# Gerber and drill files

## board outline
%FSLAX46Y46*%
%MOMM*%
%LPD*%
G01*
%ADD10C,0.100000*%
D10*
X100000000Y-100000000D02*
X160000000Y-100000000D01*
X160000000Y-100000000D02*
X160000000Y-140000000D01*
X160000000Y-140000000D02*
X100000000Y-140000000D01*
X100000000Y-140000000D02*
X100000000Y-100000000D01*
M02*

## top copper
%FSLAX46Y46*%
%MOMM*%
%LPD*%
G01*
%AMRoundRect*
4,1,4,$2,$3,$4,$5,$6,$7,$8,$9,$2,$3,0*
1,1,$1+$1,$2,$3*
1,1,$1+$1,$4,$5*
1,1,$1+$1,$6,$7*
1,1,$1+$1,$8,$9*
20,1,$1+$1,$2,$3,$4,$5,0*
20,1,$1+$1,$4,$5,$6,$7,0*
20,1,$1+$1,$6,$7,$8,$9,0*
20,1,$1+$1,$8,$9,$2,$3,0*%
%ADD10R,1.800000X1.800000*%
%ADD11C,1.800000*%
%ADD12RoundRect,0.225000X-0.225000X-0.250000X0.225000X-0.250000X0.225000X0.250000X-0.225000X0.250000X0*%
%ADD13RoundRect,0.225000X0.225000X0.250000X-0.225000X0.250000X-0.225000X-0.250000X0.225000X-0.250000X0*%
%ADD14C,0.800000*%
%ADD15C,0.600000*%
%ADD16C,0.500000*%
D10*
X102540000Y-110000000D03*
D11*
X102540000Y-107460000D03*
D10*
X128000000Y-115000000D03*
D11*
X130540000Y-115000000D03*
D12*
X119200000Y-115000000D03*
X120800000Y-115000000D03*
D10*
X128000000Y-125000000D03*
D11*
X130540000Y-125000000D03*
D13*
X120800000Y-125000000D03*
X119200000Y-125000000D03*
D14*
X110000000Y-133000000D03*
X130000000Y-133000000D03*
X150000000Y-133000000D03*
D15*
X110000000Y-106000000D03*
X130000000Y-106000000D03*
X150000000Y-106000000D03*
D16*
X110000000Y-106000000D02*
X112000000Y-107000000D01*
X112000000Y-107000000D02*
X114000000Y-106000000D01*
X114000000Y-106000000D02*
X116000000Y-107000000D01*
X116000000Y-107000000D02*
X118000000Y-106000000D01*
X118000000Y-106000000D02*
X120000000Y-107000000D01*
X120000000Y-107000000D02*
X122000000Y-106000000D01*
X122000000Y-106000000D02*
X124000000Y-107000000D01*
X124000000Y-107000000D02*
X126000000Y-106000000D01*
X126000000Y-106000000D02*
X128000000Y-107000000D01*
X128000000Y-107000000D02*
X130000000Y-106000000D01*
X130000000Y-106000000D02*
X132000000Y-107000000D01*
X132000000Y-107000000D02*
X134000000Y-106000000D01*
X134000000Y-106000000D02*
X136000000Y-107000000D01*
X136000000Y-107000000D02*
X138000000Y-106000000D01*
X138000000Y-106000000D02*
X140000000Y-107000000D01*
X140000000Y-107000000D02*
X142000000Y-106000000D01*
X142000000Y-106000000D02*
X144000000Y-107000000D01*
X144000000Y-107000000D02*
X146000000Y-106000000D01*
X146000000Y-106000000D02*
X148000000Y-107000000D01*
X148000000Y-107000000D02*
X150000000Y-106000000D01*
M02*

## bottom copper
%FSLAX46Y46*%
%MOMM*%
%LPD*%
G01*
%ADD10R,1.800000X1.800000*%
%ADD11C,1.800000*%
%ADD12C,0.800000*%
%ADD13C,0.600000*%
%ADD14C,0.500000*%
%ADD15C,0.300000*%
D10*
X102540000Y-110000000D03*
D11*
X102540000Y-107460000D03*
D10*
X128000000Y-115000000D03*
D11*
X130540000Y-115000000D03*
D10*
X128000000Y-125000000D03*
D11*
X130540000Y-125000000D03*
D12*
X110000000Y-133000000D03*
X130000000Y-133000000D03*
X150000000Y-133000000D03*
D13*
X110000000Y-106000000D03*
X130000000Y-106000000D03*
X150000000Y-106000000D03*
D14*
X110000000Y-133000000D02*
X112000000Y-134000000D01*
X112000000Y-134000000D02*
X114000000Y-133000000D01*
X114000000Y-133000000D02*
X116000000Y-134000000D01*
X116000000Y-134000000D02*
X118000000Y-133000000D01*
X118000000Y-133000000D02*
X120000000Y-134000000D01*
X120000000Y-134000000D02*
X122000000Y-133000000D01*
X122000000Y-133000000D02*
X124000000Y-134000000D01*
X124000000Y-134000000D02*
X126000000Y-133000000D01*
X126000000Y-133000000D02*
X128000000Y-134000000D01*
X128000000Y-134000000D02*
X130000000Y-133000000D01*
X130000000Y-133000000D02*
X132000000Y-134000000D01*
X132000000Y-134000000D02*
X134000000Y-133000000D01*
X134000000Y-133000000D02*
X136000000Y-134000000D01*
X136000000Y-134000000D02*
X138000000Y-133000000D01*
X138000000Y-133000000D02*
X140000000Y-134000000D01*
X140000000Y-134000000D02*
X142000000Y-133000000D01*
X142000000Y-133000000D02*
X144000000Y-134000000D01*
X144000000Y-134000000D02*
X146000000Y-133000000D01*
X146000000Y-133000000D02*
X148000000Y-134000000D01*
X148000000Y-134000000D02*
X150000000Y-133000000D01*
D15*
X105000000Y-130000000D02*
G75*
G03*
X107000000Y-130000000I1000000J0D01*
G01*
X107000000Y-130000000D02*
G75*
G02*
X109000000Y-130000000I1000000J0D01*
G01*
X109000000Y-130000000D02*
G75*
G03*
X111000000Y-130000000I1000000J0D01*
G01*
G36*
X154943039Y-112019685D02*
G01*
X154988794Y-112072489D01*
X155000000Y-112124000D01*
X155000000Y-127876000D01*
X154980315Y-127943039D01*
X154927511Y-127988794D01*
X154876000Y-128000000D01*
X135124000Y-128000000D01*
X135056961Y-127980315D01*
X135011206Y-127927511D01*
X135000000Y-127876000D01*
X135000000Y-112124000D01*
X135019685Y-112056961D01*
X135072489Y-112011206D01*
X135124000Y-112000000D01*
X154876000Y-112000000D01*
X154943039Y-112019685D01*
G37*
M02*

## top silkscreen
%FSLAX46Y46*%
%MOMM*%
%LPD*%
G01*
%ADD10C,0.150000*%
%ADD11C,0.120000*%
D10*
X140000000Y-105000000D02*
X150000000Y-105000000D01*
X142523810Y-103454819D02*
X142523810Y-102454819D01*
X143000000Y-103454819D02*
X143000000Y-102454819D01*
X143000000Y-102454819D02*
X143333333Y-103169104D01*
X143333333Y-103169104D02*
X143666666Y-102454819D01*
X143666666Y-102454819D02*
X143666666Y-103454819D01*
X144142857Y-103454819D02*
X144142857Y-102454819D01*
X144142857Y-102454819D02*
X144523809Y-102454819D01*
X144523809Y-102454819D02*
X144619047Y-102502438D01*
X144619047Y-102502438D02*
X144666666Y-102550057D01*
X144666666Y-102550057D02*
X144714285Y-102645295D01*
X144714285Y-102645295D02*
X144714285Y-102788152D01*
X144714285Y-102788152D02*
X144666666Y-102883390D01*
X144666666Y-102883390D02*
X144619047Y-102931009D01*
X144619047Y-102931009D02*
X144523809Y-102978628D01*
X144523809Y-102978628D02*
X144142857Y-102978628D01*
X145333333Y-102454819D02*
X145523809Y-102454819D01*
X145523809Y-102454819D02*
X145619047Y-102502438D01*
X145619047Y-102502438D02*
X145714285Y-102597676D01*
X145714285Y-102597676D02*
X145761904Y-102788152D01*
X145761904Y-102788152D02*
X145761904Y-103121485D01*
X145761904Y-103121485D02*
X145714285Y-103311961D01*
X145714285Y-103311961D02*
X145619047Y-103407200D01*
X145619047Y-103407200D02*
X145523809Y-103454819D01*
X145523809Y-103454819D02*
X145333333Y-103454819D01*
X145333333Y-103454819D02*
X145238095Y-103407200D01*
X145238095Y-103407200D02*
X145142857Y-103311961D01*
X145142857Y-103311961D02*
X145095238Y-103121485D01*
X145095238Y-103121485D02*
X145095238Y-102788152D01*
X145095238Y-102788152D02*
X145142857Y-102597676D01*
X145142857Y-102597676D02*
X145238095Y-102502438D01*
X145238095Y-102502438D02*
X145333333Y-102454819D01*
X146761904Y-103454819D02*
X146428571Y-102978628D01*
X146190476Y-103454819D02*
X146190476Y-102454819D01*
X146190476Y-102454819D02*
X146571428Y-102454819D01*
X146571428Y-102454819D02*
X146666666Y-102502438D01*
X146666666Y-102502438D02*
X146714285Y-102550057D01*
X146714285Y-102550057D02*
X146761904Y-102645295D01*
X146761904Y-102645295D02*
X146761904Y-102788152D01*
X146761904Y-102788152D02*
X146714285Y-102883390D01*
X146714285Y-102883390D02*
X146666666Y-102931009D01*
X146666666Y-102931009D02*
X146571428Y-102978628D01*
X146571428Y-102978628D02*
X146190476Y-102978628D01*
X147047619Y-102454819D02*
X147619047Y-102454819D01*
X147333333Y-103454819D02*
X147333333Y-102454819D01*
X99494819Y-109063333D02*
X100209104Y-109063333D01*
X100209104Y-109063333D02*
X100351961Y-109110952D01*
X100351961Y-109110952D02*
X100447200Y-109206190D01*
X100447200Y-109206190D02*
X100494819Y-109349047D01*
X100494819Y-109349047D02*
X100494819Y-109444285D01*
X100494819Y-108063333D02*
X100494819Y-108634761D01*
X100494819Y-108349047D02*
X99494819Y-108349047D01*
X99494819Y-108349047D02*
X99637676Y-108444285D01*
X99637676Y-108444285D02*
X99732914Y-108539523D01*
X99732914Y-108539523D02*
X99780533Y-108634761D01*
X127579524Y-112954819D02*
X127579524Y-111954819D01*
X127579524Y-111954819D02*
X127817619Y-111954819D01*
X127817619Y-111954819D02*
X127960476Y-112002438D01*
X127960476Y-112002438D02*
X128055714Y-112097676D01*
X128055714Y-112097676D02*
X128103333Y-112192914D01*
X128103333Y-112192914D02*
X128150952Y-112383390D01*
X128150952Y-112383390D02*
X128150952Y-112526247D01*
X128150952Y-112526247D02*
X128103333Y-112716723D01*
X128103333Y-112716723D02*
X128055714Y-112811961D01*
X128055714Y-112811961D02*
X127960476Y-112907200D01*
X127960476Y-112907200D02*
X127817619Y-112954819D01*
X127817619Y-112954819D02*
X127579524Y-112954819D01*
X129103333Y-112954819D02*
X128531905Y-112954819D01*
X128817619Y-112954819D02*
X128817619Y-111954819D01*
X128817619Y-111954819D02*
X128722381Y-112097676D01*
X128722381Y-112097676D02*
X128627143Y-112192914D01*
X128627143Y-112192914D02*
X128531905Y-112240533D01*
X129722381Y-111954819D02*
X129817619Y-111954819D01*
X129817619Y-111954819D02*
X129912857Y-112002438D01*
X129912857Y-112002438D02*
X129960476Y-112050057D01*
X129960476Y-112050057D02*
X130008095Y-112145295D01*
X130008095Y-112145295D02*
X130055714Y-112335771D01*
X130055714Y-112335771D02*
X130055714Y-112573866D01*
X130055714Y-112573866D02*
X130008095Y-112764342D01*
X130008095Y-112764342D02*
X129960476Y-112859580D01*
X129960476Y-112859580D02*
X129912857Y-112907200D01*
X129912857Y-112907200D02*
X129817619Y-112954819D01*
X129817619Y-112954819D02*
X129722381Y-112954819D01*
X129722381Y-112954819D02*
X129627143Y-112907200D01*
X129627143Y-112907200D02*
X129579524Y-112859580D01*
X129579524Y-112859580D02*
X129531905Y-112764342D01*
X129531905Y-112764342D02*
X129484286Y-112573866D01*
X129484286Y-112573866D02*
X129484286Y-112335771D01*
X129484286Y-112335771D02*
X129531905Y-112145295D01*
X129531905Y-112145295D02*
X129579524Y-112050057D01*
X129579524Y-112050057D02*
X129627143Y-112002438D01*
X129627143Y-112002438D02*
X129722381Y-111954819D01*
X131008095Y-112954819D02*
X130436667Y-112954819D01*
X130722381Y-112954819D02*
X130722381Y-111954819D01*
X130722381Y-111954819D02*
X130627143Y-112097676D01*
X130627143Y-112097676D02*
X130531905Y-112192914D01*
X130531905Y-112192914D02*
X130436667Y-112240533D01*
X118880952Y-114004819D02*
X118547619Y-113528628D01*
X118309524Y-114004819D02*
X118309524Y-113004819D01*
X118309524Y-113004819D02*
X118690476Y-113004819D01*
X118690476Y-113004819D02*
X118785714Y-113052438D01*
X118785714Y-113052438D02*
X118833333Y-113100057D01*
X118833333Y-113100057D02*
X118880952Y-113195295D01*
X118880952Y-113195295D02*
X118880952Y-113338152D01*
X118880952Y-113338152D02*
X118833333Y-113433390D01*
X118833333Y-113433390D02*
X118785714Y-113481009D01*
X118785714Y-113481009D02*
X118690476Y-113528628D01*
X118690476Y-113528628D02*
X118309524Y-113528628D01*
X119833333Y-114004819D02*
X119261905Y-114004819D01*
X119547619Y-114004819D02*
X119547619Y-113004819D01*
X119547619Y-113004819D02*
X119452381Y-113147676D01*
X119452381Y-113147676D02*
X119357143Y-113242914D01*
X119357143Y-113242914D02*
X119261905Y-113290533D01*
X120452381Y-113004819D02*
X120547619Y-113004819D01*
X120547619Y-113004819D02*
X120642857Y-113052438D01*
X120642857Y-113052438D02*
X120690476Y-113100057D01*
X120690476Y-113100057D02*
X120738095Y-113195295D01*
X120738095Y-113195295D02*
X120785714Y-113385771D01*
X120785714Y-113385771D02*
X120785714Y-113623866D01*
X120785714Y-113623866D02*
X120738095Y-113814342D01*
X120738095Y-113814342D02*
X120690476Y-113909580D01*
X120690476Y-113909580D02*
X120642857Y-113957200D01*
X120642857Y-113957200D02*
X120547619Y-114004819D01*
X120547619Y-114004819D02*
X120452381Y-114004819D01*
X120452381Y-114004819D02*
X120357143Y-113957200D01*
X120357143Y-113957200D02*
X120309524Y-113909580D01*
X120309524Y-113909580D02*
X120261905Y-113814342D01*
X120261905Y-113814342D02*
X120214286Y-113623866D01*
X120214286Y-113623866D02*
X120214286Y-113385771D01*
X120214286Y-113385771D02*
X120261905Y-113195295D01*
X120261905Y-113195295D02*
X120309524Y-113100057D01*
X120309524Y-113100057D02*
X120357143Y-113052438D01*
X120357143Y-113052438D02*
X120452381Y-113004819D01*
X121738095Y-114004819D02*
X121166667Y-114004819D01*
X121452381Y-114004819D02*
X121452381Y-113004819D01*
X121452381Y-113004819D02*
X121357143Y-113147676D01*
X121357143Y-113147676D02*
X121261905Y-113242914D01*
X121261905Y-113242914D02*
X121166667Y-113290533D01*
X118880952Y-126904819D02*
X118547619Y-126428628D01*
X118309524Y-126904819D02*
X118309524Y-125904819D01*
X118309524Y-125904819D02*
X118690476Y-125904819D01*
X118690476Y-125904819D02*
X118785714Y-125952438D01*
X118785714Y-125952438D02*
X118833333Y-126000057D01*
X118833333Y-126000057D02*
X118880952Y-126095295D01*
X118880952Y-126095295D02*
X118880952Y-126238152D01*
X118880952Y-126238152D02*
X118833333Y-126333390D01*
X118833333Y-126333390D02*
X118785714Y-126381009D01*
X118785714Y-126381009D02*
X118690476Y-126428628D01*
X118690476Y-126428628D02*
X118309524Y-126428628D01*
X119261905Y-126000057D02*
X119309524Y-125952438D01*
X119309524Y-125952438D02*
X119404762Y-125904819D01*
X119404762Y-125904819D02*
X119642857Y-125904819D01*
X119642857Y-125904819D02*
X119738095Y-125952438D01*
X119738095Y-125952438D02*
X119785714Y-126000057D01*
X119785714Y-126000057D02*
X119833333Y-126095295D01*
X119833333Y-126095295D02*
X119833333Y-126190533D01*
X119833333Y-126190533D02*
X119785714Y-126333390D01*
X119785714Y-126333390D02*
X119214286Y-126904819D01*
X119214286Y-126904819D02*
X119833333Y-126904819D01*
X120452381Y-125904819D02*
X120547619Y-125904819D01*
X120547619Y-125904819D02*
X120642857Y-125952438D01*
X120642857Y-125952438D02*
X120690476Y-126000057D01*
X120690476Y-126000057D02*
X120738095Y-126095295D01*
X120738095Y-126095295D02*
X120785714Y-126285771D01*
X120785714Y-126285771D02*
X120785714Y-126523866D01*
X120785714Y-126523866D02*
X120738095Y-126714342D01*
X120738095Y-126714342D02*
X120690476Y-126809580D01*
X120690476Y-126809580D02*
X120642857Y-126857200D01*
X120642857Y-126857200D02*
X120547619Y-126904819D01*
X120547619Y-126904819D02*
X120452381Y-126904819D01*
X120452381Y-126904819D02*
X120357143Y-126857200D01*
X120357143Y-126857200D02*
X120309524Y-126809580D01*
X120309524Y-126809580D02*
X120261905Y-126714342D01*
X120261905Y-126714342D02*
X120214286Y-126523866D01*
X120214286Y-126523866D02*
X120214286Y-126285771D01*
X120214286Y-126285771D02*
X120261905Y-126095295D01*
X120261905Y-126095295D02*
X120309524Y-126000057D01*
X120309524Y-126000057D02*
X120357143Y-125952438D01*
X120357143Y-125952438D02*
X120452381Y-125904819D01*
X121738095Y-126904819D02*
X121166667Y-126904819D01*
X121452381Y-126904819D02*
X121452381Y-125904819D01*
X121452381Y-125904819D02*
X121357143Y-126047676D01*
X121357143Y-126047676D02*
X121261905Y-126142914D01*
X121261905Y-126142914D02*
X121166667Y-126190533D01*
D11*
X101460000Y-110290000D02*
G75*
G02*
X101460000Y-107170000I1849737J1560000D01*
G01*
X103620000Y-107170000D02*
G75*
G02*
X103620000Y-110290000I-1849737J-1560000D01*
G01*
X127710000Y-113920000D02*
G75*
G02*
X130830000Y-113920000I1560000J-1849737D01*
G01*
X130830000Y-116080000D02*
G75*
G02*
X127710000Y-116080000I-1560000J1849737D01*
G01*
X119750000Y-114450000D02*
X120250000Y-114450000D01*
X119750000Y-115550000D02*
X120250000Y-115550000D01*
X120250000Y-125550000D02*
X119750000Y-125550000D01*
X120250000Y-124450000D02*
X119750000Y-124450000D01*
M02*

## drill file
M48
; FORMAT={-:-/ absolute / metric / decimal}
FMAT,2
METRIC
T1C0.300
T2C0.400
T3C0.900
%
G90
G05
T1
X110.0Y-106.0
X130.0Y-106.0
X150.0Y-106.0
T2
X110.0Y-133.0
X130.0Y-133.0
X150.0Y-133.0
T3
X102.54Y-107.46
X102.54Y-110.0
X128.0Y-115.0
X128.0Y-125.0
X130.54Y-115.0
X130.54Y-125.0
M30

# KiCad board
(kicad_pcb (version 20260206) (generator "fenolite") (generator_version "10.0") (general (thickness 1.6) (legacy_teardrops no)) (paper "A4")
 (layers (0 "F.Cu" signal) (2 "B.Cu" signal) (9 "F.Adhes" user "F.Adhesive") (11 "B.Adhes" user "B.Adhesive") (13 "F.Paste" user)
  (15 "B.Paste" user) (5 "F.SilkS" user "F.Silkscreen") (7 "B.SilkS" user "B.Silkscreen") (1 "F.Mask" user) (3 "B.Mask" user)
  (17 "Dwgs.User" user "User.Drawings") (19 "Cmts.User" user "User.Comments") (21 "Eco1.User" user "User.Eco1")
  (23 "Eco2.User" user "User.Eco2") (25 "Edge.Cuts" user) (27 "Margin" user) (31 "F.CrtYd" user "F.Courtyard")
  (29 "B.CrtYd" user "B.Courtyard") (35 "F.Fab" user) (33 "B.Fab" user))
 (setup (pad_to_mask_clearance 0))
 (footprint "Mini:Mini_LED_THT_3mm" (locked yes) (layer "F.Cu") (at 102.54 110 90)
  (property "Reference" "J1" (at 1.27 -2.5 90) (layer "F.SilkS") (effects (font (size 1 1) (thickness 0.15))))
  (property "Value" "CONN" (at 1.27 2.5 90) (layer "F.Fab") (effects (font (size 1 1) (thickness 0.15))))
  (fp_arc (start -0.29 -1.08) (mid 1.27 -1.65) (end 2.83 -1.08) (stroke (width 0.12) (type solid)) (layer "F.SilkS"))
  (fp_arc (start 2.83 1.08) (mid 1.27 1.65) (end -0.29 1.08) (stroke (width 0.12) (type solid)) (layer "F.SilkS"))
  (pad "1" thru_hole rect (at 0 0 90) (size 1.8 1.8) (drill 0.9) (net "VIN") (layers "*.Cu" "*.Mask") (remove_unused_layers no))
  (pad "2" thru_hole circle (at 2.54 0 90) (size 1.8 1.8) (drill 0.9) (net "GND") (layers "*.Cu" "*.Mask") (remove_unused_layers no)))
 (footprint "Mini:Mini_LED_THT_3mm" (layer "F.Cu") (at 128 115)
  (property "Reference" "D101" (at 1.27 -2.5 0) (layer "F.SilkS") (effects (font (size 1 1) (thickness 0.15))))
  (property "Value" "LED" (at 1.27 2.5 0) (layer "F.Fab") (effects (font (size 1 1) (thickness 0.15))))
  (fp_arc (start -0.29 -1.08) (mid 1.27 -1.65) (end 2.83 -1.08) (stroke (width 0.12) (type solid)) (layer "F.SilkS"))
  (fp_arc (start 2.83 1.08) (mid 1.27 1.65) (end -0.29 1.08) (stroke (width 0.12) (type solid)) (layer "F.SilkS"))
  (pad "1" thru_hole rect (at 0 0) (size 1.8 1.8) (drill 0.9) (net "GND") (layers "*.Cu" "*.Mask") (remove_unused_layers no))
  (pad "2" thru_hole circle (at 2.54 0) (size 1.8 1.8) (drill 0.9) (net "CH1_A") (layers "*.Cu" "*.Mask") (remove_unused_layers no)))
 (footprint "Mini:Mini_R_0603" (layer "F.Cu") (at 120 115)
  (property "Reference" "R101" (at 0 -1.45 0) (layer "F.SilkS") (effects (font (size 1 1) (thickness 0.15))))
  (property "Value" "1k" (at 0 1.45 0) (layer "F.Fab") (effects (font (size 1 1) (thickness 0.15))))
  (fp_line (start -0.25 -0.55) (end 0.25 -0.55) (stroke (width 0.12) (type solid)) (layer "F.SilkS"))
  (fp_line (start -0.25 0.55) (end 0.25 0.55) (stroke (width 0.12) (type solid)) (layer "F.SilkS"))
  (pad "1" smd roundrect (at -0.8 0) (size 0.9 0.95) (layers "F.Cu" "F.Mask" "F.Paste") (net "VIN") (roundrect_rratio 0.25))
  (pad "2" smd roundrect (at 0.8 0) (size 0.9 0.95) (layers "F.Cu" "F.Mask" "F.Paste") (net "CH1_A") (roundrect_rratio 0.25)))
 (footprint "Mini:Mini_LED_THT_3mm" (layer "B.Cu") (at 128 125)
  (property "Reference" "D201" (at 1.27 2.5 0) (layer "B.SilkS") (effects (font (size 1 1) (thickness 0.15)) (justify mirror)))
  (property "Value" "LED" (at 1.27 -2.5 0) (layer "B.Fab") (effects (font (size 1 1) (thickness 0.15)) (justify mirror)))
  (pad "1" thru_hole rect (at 0 0) (size 1.8 1.8) (drill 0.9) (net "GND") (layers "*.Cu" "*.Mask") (remove_unused_layers no))
  (pad "2" thru_hole circle (at 2.54 0) (size 1.8 1.8) (drill 0.9) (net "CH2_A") (layers "*.Cu" "*.Mask") (remove_unused_layers no)))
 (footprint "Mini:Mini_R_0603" (layer "F.Cu") (at 120 125 180)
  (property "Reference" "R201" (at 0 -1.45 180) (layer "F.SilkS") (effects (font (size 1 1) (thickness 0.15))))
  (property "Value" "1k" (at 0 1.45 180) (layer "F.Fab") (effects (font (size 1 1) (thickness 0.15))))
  (fp_line (start -0.25 -0.55) (end 0.25 -0.55) (stroke (width 0.12) (type solid)) (layer "F.SilkS"))
  (fp_line (start -0.25 0.55) (end 0.25 0.55) (stroke (width 0.12) (type solid)) (layer "F.SilkS"))
  (pad "1" smd roundrect (at -0.8 0 180) (size 0.9 0.95) (layers "F.Cu" "F.Mask" "F.Paste") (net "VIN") (roundrect_rratio 0.25))
  (pad "2" smd roundrect (at 0.8 0 180) (size 0.9 0.95) (layers "F.Cu" "F.Mask" "F.Paste") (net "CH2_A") (roundrect_rratio 0.25)))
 (gr_line (start 140 105) (end 150 105) (stroke (width 0.15) (type solid)) (layer "F.SilkS"))
 (gr_line (start 100 100) (end 160 100) (stroke (width 0.1) (type solid)) (layer "Edge.Cuts"))
 (gr_line (start 160 100) (end 160 140) (stroke (width 0.1) (type solid)) (layer "Edge.Cuts"))
 (gr_line (start 160 140) (end 100 140) (stroke (width 0.1) (type solid)) (layer "Edge.Cuts"))
 (gr_line (start 100 140) (end 100 100) (stroke (width 0.1) (type solid)) (layer "Edge.Cuts"))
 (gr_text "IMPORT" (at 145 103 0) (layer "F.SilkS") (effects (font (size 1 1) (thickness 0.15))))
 (segment (start 110 133) (end 112 134) (width 0.5) (locked yes) (layer "B.Cu") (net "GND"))
 (segment (start 112 134) (end 114 133) (width 0.5) (locked yes) (layer "B.Cu") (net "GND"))
 (segment (start 114 133) (end 116 134) (width 0.5) (locked yes) (layer "B.Cu") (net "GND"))
 (segment (start 116 134) (end 118 133) (width 0.5) (locked yes) (layer "B.Cu") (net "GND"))
 (segment (start 118 133) (end 120 134) (width 0.5) (locked yes) (layer "B.Cu") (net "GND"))
 (segment (start 120 134) (end 122 133) (width 0.5) (locked yes) (layer "B.Cu") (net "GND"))
 (segment (start 122 133) (end 124 134) (width 0.5) (locked yes) (layer "B.Cu") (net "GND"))
 (segment (start 124 134) (end 126 133) (width 0.5) (locked yes) (layer "B.Cu") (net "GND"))
 (segment (start 126 133) (end 128 134) (width 0.5) (locked yes) (layer "B.Cu") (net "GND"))
 (segment (start 128 134) (end 130 133) (width 0.5) (locked yes) (layer "B.Cu") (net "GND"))
 (segment (start 130 133) (end 132 134) (width 0.5) (locked yes) (layer "B.Cu") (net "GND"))
 (segment (start 132 134) (end 134 133) (width 0.5) (locked yes) (layer "B.Cu") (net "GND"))
 (segment (start 134 133) (end 136 134) (width 0.5) (locked yes) (layer "B.Cu") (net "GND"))
 (segment (start 136 134) (end 138 133) (width 0.5) (locked yes) (layer "B.Cu") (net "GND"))
 (segment (start 138 133) (end 140 134) (width 0.5) (locked yes) (layer "B.Cu") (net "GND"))
 (segment (start 140 134) (end 142 133) (width 0.5) (locked yes) (layer "B.Cu") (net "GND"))
 (segment (start 142 133) (end 144 134) (width 0.5) (locked yes) (layer "B.Cu") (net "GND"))
 (segment (start 144 134) (end 146 133) (width 0.5) (locked yes) (layer "B.Cu") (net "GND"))
 (segment (start 146 133) (end 148 134) (width 0.5) (locked yes) (layer "B.Cu") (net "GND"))
 (segment (start 148 134) (end 150 133) (width 0.5) (locked yes) (layer "B.Cu") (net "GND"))
 (segment (start 110 106) (end 112 107) (width 0.5) (layer "F.Cu") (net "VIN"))
 (segment (start 112 107) (end 114 106) (width 0.5) (layer "F.Cu") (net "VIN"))
 (segment (start 114 106) (end 116 107) (width 0.5) (layer "F.Cu") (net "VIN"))
 (segment (start 116 107) (end 118 106) (width 0.5) (layer "F.Cu") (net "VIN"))
 (segment (start 118 106) (end 120 107) (width 0.5) (layer "F.Cu") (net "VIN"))
 (segment (start 120 107) (end 122 106) (width 0.5) (layer "F.Cu") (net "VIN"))
 (segment (start 122 106) (end 124 107) (width 0.5) (layer "F.Cu") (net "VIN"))
 (segment (start 124 107) (end 126 106) (width 0.5) (layer "F.Cu") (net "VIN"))
 (segment (start 126 106) (end 128 107) (width 0.5) (layer "F.Cu") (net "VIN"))
 (segment (start 128 107) (end 130 106) (width 0.5) (layer "F.Cu") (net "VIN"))
 (segment (start 130 106) (end 132 107) (width 0.5) (layer "F.Cu") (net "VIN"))
 (segment (start 132 107) (end 134 106) (width 0.5) (layer "F.Cu") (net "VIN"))
 (segment (start 134 106) (end 136 107) (width 0.5) (layer "F.Cu") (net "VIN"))
 (segment (start 136 107) (end 138 106) (width 0.5) (layer "F.Cu") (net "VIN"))
 (segment (start 138 106) (end 140 107) (width 0.5) (layer "F.Cu") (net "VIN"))
 (segment (start 140 107) (end 142 106) (width 0.5) (layer "F.Cu") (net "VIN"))
 (segment (start 142 106) (end 144 107) (width 0.5) (layer "F.Cu") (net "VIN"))
 (segment (start 144 107) (end 146 106) (width 0.5) (layer "F.Cu") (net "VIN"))
 (segment (start 146 106) (end 148 107) (width 0.5) (layer "F.Cu") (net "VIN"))
 (segment (start 148 107) (end 150 106) (width 0.5) (layer "F.Cu") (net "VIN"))
 (arc (start 105 130) (mid 106 131) (end 107 130) (width 0.3) (layer "B.Cu") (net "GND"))
 (arc (start 107 130) (mid 108 129) (end 109 130) (width 0.3) (layer "B.Cu") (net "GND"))
 (arc (start 109 130) (mid 110 131) (end 111 130) (width 0.3) (layer "B.Cu") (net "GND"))
 (via (at 110 133) (size 0.8) (drill 0.4) (layers "F.Cu" "B.Cu") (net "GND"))
 (via (at 130 133) (size 0.8) (drill 0.4) (layers "F.Cu" "B.Cu") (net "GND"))
 (via (at 150 133) (size 0.8) (drill 0.4) (layers "F.Cu" "B.Cu") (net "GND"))
 (via (at 110 106) (size 0.6) (drill 0.3) (layers "F.Cu" "B.Cu") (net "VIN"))
 (via (at 130 106) (size 0.6) (drill 0.3) (layers "F.Cu" "B.Cu") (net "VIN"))
 (via (at 150 106) (size 0.6) (drill 0.3) (layers "F.Cu" "B.Cu") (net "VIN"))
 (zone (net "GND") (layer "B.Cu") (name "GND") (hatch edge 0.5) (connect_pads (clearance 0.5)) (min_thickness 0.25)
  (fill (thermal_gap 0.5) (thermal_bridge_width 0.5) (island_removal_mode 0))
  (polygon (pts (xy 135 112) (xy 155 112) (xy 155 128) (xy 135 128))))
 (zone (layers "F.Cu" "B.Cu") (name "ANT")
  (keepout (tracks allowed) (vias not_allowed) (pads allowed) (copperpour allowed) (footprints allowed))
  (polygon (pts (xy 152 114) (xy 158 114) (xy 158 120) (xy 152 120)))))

